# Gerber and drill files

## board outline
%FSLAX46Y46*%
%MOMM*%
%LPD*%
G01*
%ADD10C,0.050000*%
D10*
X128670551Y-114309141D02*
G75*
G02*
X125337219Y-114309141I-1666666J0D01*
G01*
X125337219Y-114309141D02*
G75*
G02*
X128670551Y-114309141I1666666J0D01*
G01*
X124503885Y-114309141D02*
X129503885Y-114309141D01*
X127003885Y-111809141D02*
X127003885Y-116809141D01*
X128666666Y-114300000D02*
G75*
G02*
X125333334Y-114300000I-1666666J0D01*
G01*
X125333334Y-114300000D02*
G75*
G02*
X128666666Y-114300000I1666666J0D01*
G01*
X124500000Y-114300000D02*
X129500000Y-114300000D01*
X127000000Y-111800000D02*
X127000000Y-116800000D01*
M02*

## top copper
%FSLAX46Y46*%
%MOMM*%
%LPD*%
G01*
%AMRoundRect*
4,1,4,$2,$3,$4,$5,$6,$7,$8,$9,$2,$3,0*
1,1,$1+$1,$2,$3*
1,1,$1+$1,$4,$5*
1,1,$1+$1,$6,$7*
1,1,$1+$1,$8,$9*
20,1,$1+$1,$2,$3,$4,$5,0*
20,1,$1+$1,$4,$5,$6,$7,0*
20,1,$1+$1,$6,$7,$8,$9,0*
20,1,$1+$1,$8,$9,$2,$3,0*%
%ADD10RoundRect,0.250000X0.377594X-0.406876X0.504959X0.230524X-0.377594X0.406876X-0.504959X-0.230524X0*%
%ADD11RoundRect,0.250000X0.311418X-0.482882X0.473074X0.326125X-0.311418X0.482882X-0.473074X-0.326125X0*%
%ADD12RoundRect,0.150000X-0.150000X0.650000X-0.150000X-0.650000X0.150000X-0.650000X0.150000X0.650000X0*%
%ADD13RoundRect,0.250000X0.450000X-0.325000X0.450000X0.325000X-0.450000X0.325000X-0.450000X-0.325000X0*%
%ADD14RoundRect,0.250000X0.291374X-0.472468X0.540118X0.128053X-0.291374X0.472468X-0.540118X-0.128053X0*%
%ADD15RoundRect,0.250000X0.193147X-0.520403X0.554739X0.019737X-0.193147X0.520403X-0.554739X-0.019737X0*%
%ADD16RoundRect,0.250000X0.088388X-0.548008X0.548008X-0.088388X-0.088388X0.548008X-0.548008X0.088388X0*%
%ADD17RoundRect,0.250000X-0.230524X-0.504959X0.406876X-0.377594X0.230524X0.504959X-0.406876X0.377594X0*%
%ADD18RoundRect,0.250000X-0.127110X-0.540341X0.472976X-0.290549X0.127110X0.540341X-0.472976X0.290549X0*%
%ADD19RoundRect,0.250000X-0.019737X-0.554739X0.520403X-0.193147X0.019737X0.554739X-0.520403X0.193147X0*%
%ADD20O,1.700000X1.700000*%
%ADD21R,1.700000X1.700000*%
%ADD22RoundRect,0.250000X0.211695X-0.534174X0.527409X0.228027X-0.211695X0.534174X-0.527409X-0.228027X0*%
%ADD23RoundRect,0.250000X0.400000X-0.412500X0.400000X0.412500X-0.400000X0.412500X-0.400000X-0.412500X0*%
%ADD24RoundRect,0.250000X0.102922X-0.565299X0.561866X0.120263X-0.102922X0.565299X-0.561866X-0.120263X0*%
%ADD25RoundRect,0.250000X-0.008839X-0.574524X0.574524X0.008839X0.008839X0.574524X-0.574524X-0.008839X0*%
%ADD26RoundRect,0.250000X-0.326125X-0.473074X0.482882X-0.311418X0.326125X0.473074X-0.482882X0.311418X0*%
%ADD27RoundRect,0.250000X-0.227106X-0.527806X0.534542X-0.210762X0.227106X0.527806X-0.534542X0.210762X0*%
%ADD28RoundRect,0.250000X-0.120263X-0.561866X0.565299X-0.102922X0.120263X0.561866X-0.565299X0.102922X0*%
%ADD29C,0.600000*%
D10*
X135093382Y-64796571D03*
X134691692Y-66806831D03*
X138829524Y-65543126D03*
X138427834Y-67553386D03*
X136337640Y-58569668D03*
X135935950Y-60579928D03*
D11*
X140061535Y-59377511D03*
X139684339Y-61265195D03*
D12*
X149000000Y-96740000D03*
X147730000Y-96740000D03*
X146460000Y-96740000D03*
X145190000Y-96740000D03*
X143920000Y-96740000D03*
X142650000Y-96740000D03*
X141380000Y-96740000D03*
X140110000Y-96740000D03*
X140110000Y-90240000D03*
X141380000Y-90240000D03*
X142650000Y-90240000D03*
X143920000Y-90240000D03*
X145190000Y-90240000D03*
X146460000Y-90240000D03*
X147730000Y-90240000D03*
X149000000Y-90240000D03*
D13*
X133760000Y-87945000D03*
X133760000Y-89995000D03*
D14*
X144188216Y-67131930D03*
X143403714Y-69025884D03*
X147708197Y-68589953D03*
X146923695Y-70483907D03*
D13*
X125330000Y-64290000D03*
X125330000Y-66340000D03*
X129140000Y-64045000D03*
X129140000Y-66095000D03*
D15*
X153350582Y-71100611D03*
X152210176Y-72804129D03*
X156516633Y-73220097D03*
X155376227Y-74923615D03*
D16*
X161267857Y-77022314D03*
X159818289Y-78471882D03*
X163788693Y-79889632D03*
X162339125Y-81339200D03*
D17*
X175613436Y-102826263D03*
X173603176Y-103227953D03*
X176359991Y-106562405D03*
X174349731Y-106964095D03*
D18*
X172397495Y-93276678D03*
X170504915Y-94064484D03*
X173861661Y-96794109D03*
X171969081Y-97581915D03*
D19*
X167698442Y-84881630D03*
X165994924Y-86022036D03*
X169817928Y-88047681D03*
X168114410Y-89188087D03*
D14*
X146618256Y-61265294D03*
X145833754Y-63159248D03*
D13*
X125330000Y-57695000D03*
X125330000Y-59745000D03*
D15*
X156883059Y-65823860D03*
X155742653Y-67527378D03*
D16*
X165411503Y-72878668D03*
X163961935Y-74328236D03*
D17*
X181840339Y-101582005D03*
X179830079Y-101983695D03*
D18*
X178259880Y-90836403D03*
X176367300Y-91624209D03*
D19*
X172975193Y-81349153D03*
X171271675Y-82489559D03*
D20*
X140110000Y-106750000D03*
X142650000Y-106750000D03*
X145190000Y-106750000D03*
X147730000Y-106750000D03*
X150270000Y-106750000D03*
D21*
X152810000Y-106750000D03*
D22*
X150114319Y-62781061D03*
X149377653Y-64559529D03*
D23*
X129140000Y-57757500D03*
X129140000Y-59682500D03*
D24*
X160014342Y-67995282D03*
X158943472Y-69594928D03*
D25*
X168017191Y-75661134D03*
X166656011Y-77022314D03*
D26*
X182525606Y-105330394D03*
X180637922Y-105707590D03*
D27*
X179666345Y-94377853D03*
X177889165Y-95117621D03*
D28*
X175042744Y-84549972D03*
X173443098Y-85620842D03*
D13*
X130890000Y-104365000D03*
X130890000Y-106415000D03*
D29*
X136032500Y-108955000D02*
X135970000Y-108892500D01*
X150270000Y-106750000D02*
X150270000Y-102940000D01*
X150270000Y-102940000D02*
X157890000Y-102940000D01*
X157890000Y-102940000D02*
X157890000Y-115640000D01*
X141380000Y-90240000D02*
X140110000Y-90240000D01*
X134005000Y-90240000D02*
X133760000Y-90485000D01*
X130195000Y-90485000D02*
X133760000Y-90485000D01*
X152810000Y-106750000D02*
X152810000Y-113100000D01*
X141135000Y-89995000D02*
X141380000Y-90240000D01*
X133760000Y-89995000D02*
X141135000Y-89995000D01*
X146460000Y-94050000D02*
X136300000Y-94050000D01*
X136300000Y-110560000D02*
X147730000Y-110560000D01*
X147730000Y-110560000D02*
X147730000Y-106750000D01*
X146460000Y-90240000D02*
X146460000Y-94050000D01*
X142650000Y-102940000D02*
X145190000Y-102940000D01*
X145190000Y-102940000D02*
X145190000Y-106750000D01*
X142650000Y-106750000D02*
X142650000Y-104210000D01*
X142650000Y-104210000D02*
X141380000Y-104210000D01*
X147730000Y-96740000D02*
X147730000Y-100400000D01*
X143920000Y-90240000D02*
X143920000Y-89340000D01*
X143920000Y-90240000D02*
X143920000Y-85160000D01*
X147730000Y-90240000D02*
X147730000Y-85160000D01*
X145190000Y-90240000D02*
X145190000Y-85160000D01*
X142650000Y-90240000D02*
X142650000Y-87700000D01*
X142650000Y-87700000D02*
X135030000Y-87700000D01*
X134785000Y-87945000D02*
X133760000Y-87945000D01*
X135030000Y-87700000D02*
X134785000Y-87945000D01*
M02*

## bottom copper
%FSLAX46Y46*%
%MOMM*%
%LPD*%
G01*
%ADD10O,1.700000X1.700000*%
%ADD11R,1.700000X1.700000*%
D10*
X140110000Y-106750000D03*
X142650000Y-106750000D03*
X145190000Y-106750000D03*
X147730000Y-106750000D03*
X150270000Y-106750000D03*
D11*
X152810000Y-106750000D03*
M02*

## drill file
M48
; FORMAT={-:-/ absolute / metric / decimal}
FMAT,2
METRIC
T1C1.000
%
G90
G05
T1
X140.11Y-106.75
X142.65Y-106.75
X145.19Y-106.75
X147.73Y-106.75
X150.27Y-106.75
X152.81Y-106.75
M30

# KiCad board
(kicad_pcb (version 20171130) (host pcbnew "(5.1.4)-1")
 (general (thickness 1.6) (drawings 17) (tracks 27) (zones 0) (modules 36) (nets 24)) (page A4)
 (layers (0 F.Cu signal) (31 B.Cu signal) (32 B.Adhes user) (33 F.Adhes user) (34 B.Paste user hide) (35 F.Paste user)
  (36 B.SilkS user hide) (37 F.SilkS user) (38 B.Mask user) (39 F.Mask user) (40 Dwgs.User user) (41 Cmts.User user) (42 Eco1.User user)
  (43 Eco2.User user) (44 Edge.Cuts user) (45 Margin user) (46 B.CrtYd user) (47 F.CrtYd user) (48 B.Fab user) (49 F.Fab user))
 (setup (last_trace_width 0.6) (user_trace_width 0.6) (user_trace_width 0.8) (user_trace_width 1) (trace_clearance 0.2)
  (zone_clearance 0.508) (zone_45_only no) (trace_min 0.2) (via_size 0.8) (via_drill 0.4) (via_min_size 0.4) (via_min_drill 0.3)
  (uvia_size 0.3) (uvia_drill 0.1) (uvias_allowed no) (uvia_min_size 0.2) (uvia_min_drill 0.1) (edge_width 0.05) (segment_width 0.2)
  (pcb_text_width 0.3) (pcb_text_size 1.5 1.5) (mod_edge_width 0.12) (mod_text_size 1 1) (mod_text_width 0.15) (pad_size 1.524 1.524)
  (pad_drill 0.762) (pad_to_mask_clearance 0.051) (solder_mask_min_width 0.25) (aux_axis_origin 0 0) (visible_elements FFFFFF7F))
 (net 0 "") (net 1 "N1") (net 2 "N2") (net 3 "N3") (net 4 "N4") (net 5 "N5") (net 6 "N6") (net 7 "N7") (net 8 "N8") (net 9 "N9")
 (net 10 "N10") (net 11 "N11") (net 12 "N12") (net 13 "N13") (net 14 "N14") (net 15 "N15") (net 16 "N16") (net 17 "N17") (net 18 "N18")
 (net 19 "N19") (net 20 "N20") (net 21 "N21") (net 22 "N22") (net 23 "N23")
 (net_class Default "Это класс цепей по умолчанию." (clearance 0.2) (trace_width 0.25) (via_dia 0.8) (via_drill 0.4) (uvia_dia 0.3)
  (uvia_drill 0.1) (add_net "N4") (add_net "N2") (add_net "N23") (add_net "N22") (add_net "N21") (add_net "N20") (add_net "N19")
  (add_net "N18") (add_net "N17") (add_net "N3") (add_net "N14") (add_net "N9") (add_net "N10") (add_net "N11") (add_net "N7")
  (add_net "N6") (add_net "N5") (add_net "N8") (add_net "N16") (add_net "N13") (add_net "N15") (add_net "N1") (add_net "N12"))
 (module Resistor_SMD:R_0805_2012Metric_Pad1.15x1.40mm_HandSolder (layer F.Cu) (at 134.892537 65.801701 78.7)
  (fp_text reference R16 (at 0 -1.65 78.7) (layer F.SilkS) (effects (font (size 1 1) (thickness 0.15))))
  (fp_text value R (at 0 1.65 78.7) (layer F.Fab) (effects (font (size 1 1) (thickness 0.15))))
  (pad 2 smd roundrect (at 1.025 0 78.7) (size 1.15 1.4) (layers F.Cu F.Paste F.Mask) (roundrect_rratio 0.217391) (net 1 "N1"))
  (pad 1 smd roundrect (at -1.025 0 78.7) (size 1.15 1.4) (layers F.Cu F.Paste F.Mask) (roundrect_rratio 0.217391) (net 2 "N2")))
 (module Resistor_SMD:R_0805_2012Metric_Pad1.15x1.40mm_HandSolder (layer F.Cu) (at 138.628679 66.548256 78.7)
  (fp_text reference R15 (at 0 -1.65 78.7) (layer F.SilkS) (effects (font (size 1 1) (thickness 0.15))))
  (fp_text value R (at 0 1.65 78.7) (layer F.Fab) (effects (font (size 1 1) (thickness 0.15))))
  (pad 2 smd roundrect (at 1.025 0 78.7) (size 1.15 1.4) (layers F.Cu F.Paste F.Mask) (roundrect_rratio 0.217391) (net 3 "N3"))
  (pad 1 smd roundrect (at -1.025 0 78.7) (size 1.15 1.4) (layers F.Cu F.Paste F.Mask) (roundrect_rratio 0.217391) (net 2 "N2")))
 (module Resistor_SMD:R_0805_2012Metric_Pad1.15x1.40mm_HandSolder (layer F.Cu) (at 136.136795 59.574798 78.7)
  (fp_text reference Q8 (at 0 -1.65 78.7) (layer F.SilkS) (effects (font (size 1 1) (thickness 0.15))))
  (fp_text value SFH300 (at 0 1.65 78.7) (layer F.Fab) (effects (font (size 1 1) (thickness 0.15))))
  (pad 2 smd roundrect (at 1.025 0 78.7) (size 1.15 1.4) (layers F.Cu F.Paste F.Mask) (roundrect_rratio 0.217391) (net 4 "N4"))
  (pad 1 smd roundrect (at -1.025 0 78.7) (size 1.15 1.4) (layers F.Cu F.Paste F.Mask) (roundrect_rratio 0.217391) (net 1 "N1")))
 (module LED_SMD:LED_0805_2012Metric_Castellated (layer F.Cu) (at 139.872937 60.321353 78.7)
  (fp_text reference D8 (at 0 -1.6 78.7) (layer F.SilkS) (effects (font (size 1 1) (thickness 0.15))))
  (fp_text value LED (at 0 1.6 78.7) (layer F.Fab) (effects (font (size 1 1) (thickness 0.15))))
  (pad 2 smd roundrect (at 0.9625 0 78.7) (size 1.325 1.3) (layers F.Cu F.Paste F.Mask) (roundrect_rratio 0.192308) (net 4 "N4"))
  (pad 1 smd roundrect (at -0.9625 0 78.7) (size 1.325 1.3) (layers F.Cu F.Paste F.Mask) (roundrect_rratio 0.192308) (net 3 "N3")))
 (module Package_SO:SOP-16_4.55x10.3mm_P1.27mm (layer F.Cu) (at 144.555 93.49 270)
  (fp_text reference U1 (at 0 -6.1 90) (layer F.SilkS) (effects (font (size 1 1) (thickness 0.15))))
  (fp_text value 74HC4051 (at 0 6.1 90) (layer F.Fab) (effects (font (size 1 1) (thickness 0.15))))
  (pad 16 smd roundrect (at 3.25 -4.445 270) (size 1.6 0.6) (layers F.Cu F.Paste F.Mask) (roundrect_rratio 0.25) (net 4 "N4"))
  (pad 15 smd roundrect (at 3.25 -3.175 270) (size 1.6 0.6) (layers F.Cu F.Paste F.Mask) (roundrect_rratio 0.25) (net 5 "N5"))
  (pad 14 smd roundrect (at 3.25 -1.905 270) (size 1.6 0.6) (layers F.Cu F.Paste F.Mask) (roundrect_rratio 0.25) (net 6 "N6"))
  (pad 13 smd roundrect (at 3.25 -0.635 270) (size 1.6 0.6) (layers F.Cu F.Paste F.Mask) (roundrect_rratio 0.25) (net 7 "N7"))
  (pad 12 smd roundrect (at 3.25 0.635 270) (size 1.6 0.6) (layers F.Cu F.Paste F.Mask) (roundrect_rratio 0.25) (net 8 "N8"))
  (pad 11 smd roundrect (at 3.25 1.905 270) (size 1.6 0.6) (layers F.Cu F.Paste F.Mask) (roundrect_rratio 0.25) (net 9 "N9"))
  (pad 10 smd roundrect (at 3.25 3.175 270) (size 1.6 0.6) (layers F.Cu F.Paste F.Mask) (roundrect_rratio 0.25) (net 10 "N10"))
  (pad 9 smd roundrect (at 3.25 4.445 270) (size 1.6 0.6) (layers F.Cu F.Paste F.Mask) (roundrect_rratio 0.25) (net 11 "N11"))
  (pad 8 smd roundrect (at -3.25 4.445 270) (size 1.6 0.6) (layers F.Cu F.Paste F.Mask) (roundrect_rratio 0.25) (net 2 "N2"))
  (pad 7 smd roundrect (at -3.25 3.175 270) (size 1.6 0.6) (layers F.Cu F.Paste F.Mask) (roundrect_rratio 0.25) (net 2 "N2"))
  (pad 6 smd roundrect (at -3.25 1.905 270) (size 1.6 0.6) (layers F.Cu F.Paste F.Mask) (roundrect_rratio 0.25) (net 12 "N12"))
  (pad 5 smd roundrect (at -3.25 0.635 270) (size 1.6 0.6) (layers F.Cu F.Paste F.Mask) (roundrect_rratio 0.25) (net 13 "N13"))
  (pad 4 smd roundrect (at -3.25 -0.635 270) (size 1.6 0.6) (layers F.Cu F.Paste F.Mask) (roundrect_rratio 0.25) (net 1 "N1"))
  (pad 3 smd roundrect (at -3.25 -1.905 270) (size 1.6 0.6) (layers F.Cu F.Paste F.Mask) (roundrect_rratio 0.25) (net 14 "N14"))
  (pad 2 smd roundrect (at -3.25 -3.175 270) (size 1.6 0.6) (layers F.Cu F.Paste F.Mask) (roundrect_rratio 0.25) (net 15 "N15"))
  (pad 1 smd roundrect (at -3.25 -4.445 270) (size 1.6 0.6) (layers F.Cu F.Paste F.Mask) (roundrect_rratio 0.25) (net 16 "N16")))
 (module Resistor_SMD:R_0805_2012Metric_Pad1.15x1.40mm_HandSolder (layer F.Cu) (at 133.76 88.97 90)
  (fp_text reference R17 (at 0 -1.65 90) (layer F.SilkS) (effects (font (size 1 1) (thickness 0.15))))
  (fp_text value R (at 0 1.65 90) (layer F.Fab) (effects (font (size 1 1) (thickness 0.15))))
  (pad 2 smd roundrect (at 1.025 0 90) (size 1.15 1.4) (layers F.Cu F.Paste F.Mask) (roundrect_rratio 0.217391) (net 12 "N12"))
  (pad 1 smd roundrect (at -1.025 0 90) (size 1.15 1.4) (layers F.Cu F.Paste F.Mask) (roundrect_rratio 0.217391) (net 2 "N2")))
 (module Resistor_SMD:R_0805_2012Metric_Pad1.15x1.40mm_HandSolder (layer F.Cu) (at 143.795965 68.078907 67.5)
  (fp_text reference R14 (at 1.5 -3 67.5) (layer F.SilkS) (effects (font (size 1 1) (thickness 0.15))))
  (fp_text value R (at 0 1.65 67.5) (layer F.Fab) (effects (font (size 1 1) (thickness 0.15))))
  (pad 2 smd roundrect (at 1.025 0 67.5) (size 1.15 1.4) (layers F.Cu F.Paste F.Mask) (roundrect_rratio 0.217391) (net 15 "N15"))
  (pad 1 smd roundrect (at -1.025 0 67.5) (size 1.15 1.4) (layers F.Cu F.Paste F.Mask) (roundrect_rratio 0.217391) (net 2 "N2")))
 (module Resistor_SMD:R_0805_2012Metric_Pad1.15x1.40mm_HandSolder (layer F.Cu) (at 147.315946 69.53693 67.5)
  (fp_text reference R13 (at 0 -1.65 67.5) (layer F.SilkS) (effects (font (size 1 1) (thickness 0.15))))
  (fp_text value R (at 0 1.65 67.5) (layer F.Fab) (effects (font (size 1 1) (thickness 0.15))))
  (pad 2 smd roundrect (at 1.025 0 67.5) (size 1.15 1.4) (layers F.Cu F.Paste F.Mask) (roundrect_rratio 0.217391) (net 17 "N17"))
  (pad 1 smd roundrect (at -1.025 0 67.5) (size 1.15 1.4) (layers F.Cu F.Paste F.Mask) (roundrect_rratio 0.217391) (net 2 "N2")))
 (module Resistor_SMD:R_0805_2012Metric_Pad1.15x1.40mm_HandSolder (layer F.Cu) (at 125.33 65.315 90)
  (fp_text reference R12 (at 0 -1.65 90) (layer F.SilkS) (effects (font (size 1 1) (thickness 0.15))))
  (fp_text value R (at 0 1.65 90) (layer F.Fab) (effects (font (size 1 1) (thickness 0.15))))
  (pad 2 smd roundrect (at 1.025 0 90) (size 1.15 1.4) (layers F.Cu F.Paste F.Mask) (roundrect_rratio 0.217391) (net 13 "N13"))
  (pad 1 smd roundrect (at -1.025 0 90) (size 1.15 1.4) (layers F.Cu F.Paste F.Mask) (roundrect_rratio 0.217391) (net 2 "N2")))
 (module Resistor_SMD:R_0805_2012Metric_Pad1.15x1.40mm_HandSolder (layer F.Cu) (at 129.14 65.07 90)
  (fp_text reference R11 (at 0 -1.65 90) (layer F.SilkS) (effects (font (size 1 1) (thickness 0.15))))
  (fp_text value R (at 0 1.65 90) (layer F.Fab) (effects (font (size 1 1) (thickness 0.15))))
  (pad 2 smd roundrect (at 1.025 0 90) (size 1.15 1.4) (layers F.Cu F.Paste F.Mask) (roundrect_rratio 0.217391) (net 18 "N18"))
  (pad 1 smd roundrect (at -1.025 0 90) (size 1.15 1.4) (layers F.Cu F.Paste F.Mask) (roundrect_rratio 0.217391) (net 2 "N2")))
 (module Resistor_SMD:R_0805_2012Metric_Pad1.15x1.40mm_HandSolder (layer F.Cu) (at 152.780379 71.95237 56.2)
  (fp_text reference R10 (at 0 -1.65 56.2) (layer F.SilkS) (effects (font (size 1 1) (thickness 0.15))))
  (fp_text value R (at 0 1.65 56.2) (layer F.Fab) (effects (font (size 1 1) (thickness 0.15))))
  (pad 2 smd roundrect (at 1.025 0 56.2) (size 1.15 1.4) (layers F.Cu F.Paste F.Mask) (roundrect_rratio 0.217391) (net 16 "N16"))
  (pad 1 smd roundrect (at -1.025 0 56.2) (size 1.15 1.4) (layers F.Cu F.Paste F.Mask) (roundrect_rratio 0.217391) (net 2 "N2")))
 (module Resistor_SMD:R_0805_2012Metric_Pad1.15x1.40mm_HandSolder (layer F.Cu) (at 155.94643 74.071856 56.2)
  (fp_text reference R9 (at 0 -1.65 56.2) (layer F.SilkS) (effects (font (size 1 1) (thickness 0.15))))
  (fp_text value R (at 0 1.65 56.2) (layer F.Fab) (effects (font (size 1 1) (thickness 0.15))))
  (pad 2 smd roundrect (at 1.025 0 56.2) (size 1.15 1.4) (layers F.Cu F.Paste F.Mask) (roundrect_rratio 0.217391) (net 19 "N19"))
  (pad 1 smd roundrect (at -1.025 0 56.2) (size 1.15 1.4) (layers F.Cu F.Paste F.Mask) (roundrect_rratio 0.217391) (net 2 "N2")))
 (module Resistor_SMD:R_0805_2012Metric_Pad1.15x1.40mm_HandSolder (layer F.Cu) (at 160.543073 77.747098 45)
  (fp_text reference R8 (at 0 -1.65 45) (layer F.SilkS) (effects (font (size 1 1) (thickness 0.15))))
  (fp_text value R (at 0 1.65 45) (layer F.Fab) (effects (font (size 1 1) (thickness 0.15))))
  (pad 2 smd roundrect (at 1.025 0 45) (size 1.15 1.4) (layers F.Cu F.Paste F.Mask) (roundrect_rratio 0.217391) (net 8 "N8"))
  (pad 1 smd roundrect (at -1.025 0 45) (size 1.15 1.4) (layers F.Cu F.Paste F.Mask) (roundrect_rratio 0.217391) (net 2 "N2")))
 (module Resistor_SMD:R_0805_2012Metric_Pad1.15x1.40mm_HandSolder (layer F.Cu) (at 163.063909 80.614416 45)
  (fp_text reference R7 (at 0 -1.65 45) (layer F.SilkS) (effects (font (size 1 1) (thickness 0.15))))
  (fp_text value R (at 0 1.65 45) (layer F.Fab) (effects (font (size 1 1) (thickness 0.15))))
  (pad 2 smd roundrect (at 1.025 0 45) (size 1.15 1.4) (layers F.Cu F.Paste F.Mask) (roundrect_rratio 0.217391) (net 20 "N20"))
  (pad 1 smd roundrect (at -1.025 0 45) (size 1.15 1.4) (layers F.Cu F.Paste F.Mask) (roundrect_rratio 0.217391) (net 2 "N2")))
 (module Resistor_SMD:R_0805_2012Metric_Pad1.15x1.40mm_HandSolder (layer F.Cu) (at 174.608306 103.027108 11.3)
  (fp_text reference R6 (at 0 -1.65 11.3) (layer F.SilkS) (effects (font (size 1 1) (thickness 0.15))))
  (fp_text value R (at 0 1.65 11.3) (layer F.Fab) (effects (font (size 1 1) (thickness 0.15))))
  (pad 2 smd roundrect (at 1.025 0 11.3) (size 1.15 1.4) (layers F.Cu F.Paste F.Mask) (roundrect_rratio 0.217391) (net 5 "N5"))
  (pad 1 smd roundrect (at -1.025 0 11.3) (size 1.15 1.4) (layers F.Cu F.Paste F.Mask) (roundrect_rratio 0.217391) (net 2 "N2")))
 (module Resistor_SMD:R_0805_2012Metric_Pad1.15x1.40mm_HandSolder (layer F.Cu) (at 175.354861 106.76325 11.3)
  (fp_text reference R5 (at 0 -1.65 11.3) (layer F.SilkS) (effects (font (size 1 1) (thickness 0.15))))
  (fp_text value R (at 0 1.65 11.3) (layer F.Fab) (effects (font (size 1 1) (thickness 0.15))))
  (pad 2 smd roundrect (at 1.025 0 11.3) (size 1.15 1.4) (layers F.Cu F.Paste F.Mask) (roundrect_rratio 0.217391) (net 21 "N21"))
  (pad 1 smd roundrect (at -1.025 0 11.3) (size 1.15 1.4) (layers F.Cu F.Paste F.Mask) (roundrect_rratio 0.217391) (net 2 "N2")))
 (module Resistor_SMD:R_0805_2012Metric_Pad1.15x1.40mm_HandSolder (layer F.Cu) (at 171.451205 93.670581 22.6)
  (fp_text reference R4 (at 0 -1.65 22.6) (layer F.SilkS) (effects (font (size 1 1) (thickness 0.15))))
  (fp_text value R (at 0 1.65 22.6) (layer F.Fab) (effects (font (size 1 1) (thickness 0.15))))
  (pad 2 smd roundrect (at 1.025 0 22.6) (size 1.15 1.4) (layers F.Cu F.Paste F.Mask) (roundrect_rratio 0.217391) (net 6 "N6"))
  (pad 1 smd roundrect (at -1.025 0 22.6) (size 1.15 1.4) (layers F.Cu F.Paste F.Mask) (roundrect_rratio 0.217391) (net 2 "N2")))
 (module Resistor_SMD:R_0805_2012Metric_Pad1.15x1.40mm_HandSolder (layer F.Cu) (at 172.915371 97.188012 22.6)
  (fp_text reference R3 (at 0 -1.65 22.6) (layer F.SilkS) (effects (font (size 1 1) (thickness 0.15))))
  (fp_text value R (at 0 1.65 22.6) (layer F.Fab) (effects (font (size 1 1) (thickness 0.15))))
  (pad 2 smd roundrect (at 1.025 0 22.6) (size 1.15 1.4) (layers F.Cu F.Paste F.Mask) (roundrect_rratio 0.217391) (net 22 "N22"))
  (pad 1 smd roundrect (at -1.025 0 22.6) (size 1.15 1.4) (layers F.Cu F.Paste F.Mask) (roundrect_rratio 0.217391) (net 2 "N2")))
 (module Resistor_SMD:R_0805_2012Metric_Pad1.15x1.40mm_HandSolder (layer F.Cu) (at 166.846683 85.451833 33.8)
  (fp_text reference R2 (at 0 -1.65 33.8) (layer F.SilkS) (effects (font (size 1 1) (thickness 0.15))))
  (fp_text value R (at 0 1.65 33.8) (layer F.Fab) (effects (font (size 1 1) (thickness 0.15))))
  (pad 2 smd roundrect (at 1.025 0 33.8) (size 1.15 1.4) (layers F.Cu F.Paste F.Mask) (roundrect_rratio 0.217391) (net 7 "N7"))
  (pad 1 smd roundrect (at -1.025 0 33.8) (size 1.15 1.4) (layers F.Cu F.Paste F.Mask) (roundrect_rratio 0.217391) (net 2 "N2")))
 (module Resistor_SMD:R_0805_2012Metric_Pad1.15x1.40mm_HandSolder (layer F.Cu) (at 168.966169 88.617884 33.8)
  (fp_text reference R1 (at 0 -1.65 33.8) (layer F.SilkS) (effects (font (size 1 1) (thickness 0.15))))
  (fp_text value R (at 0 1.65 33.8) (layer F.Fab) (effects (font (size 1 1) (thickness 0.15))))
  (pad 2 smd roundrect (at 1.025 0 33.8) (size 1.15 1.4) (layers F.Cu F.Paste F.Mask) (roundrect_rratio 0.217391) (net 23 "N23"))
  (pad 1 smd roundrect (at -1.025 0 33.8) (size 1.15 1.4) (layers F.Cu F.Paste F.Mask) (roundrect_rratio 0.217391) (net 2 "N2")))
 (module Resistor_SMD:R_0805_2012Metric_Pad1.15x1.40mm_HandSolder (layer F.Cu) (at 146.226005 62.212271 67.5)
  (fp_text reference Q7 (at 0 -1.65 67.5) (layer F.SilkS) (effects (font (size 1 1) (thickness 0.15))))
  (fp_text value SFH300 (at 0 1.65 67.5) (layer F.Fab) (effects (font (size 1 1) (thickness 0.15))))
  (pad 2 smd roundrect (at 1.025 0 67.5) (size 1.15 1.4) (layers F.Cu F.Paste F.Mask) (roundrect_rratio 0.217391) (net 4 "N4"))
  (pad 1 smd roundrect (at -1.025 0 67.5) (size 1.15 1.4) (layers F.Cu F.Paste F.Mask) (roundrect_rratio 0.217391) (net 15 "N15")))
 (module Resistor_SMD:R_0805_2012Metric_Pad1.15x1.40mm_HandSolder (layer F.Cu) (at 125.33 58.72 90)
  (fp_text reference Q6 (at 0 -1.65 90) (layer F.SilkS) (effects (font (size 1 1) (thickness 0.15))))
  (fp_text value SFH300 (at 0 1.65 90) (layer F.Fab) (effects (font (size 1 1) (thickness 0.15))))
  (pad 2 smd roundrect (at 1.025 0 90) (size 1.15 1.4) (layers F.Cu F.Paste F.Mask) (roundrect_rratio 0.217391) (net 4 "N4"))
  (pad 1 smd roundrect (at -1.025 0 90) (size 1.15 1.4) (layers F.Cu F.Paste F.Mask) (roundrect_rratio 0.217391) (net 13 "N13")))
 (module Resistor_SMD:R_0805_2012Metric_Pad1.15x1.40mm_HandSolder (layer F.Cu) (at 156.312856 66.675619 56.2)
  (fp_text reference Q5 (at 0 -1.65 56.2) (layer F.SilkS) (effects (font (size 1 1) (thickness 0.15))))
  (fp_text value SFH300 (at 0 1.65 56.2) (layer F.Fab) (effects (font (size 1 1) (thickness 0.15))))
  (pad 2 smd roundrect (at 1.025 0 56.2) (size 1.15 1.4) (layers F.Cu F.Paste F.Mask) (roundrect_rratio 0.217391) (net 4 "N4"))
  (pad 1 smd roundrect (at -1.025 0 56.2) (size 1.15 1.4) (layers F.Cu F.Paste F.Mask) (roundrect_rratio 0.217391) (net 16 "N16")))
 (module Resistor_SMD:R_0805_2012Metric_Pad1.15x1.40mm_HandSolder (layer F.Cu) (at 164.686719 73.603452 45)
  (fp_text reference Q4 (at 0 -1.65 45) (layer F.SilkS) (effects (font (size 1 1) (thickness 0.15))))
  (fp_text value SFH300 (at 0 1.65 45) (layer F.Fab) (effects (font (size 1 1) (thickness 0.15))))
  (pad 2 smd roundrect (at 1.025 0 45) (size 1.15 1.4) (layers F.Cu F.Paste F.Mask) (roundrect_rratio 0.217391) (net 4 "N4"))
  (pad 1 smd roundrect (at -1.025 0 45) (size 1.15 1.4) (layers F.Cu F.Paste F.Mask) (roundrect_rratio 0.217391) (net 8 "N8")))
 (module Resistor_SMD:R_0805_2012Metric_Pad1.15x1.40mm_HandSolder (layer F.Cu) (at 180.835209 101.78285 11.3)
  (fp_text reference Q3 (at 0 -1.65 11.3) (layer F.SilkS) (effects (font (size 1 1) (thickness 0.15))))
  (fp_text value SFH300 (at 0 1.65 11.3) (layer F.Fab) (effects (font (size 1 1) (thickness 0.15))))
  (pad 2 smd roundrect (at 1.025 0 11.3) (size 1.15 1.4) (layers F.Cu F.Paste F.Mask) (roundrect_rratio 0.217391) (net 4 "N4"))
  (pad 1 smd roundrect (at -1.025 0 11.3) (size 1.15 1.4) (layers F.Cu F.Paste F.Mask) (roundrect_rratio 0.217391) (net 5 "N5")))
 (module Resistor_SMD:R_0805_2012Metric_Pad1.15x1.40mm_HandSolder (layer F.Cu) (at 177.31359 91.230306 22.6)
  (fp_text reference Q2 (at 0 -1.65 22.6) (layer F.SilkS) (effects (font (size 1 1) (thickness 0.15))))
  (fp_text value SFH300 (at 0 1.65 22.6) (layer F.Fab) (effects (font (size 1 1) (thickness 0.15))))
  (pad 2 smd roundrect (at 1.025 0 22.6) (size 1.15 1.4) (layers F.Cu F.Paste F.Mask) (roundrect_rratio 0.217391) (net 4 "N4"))
  (pad 1 smd roundrect (at -1.025 0 22.6) (size 1.15 1.4) (layers F.Cu F.Paste F.Mask) (roundrect_rratio 0.217391) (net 6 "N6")))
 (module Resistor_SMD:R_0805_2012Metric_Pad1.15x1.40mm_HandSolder (layer F.Cu) (at 172.123434 81.919356 33.8)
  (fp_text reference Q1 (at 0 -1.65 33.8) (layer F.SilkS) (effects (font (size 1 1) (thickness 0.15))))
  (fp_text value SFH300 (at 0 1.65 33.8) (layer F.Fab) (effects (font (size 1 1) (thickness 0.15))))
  (pad 2 smd roundrect (at 1.025 0 33.8) (size 1.15 1.4) (layers F.Cu F.Paste F.Mask) (roundrect_rratio 0.217391) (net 4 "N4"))
  (pad 1 smd roundrect (at -1.025 0 33.8) (size 1.15 1.4) (layers F.Cu F.Paste F.Mask) (roundrect_rratio 0.217391) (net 7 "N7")))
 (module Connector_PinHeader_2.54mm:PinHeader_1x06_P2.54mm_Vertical (layer F.Cu) (at 152.81 106.75 270)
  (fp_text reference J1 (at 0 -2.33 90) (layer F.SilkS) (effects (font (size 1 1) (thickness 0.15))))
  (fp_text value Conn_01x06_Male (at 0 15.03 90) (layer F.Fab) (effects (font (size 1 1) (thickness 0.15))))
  (pad 6 thru_hole oval (at 0 12.7 270) (size 1.7 1.7) (drill 1) (layers *.Cu *.Mask) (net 11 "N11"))
  (pad 5 thru_hole oval (at 0 10.16 270) (size 1.7 1.7) (drill 1) (layers *.Cu *.Mask) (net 10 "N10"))
  (pad 4 thru_hole oval (at 0 7.62 270) (size 1.7 1.7) (drill 1) (layers *.Cu *.Mask) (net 9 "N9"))
  (pad 3 thru_hole oval (at 0 5.08 270) (size 1.7 1.7) (drill 1) (layers *.Cu *.Mask) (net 14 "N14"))
  (pad 2 thru_hole oval (at 0 2.54 270) (size 1.7 1.7) (drill 1) (layers *.Cu *.Mask) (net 4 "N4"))
  (pad 1 thru_hole rect (at 0 0 270) (size 1.7 1.7) (drill 1) (layers *.Cu *.Mask) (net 2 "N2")))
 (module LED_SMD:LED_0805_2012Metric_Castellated (layer F.Cu) (at 149.745986 63.670295 67.5)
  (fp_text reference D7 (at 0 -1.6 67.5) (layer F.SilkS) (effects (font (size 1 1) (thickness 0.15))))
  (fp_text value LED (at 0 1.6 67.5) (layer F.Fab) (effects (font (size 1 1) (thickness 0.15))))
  (pad 2 smd roundrect (at 0.9625 0 67.5) (size 1.325 1.3) (layers F.Cu F.Paste F.Mask) (roundrect_rratio 0.192308) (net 4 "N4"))
  (pad 1 smd roundrect (at -0.9625 0 67.5) (size 1.325 1.3) (layers F.Cu F.Paste F.Mask) (roundrect_rratio 0.192308) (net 17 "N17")))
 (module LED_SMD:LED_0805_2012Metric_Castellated (layer F.Cu) (at 129.14 58.72 90)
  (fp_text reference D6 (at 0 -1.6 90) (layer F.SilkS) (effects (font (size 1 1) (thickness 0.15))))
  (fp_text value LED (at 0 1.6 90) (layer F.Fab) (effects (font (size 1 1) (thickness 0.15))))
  (pad 2 smd roundrect (at 0.9625 0 90) (size 1.325 1.3) (layers F.Cu F.Paste F.Mask) (roundrect_rratio 0.192308) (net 4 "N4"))
  (pad 1 smd roundrect (at -0.9625 0 90) (size 1.325 1.3) (layers F.Cu F.Paste F.Mask) (roundrect_rratio 0.192308) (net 18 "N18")))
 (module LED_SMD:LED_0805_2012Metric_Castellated (layer F.Cu) (at 159.478907 68.795105 56.2)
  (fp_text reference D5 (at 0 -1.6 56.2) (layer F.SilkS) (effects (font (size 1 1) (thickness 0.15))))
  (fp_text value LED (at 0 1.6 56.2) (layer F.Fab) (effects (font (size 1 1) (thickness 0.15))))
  (pad 2 smd roundrect (at 0.9625 0 56.2) (size 1.325 1.3) (layers F.Cu F.Paste F.Mask) (roundrect_rratio 0.192308) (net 4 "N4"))
  (pad 1 smd roundrect (at -0.9625 0 56.2) (size 1.325 1.3) (layers F.Cu F.Paste F.Mask) (roundrect_rratio 0.192308) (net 19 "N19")))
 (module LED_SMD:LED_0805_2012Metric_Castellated (layer F.Cu) (at 167.336601 76.341724 45)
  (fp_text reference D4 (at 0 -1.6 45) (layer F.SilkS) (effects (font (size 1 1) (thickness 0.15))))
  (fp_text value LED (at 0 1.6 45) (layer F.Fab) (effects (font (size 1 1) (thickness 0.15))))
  (pad 2 smd roundrect (at 0.9625 0 45) (size 1.325 1.3) (layers F.Cu F.Paste F.Mask) (roundrect_rratio 0.192308) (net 4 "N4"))
  (pad 1 smd roundrect (at -0.9625 0 45) (size 1.325 1.3) (layers F.Cu F.Paste F.Mask) (roundrect_rratio 0.192308) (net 20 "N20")))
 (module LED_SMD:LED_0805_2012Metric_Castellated (layer F.Cu) (at 181.581764 105.518992 11.3)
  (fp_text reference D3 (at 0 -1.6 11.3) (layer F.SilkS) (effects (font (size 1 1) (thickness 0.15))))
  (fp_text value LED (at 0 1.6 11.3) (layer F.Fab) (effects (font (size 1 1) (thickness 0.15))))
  (pad 2 smd roundrect (at 0.9625 0 11.3) (size 1.325 1.3) (layers F.Cu F.Paste F.Mask) (roundrect_rratio 0.192308) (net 4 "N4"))
  (pad 1 smd roundrect (at -0.9625 0 11.3) (size 1.325 1.3) (layers F.Cu F.Paste F.Mask) (roundrect_rratio 0.192308) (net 21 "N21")))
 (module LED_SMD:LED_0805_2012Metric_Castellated (layer F.Cu) (at 178.777755 94.747737 22.6)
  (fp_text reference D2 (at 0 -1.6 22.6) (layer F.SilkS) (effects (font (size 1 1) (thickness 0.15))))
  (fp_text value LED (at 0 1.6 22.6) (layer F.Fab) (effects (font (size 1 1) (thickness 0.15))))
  (pad 2 smd roundrect (at 0.9625 0 22.6) (size 1.325 1.3) (layers F.Cu F.Paste F.Mask) (roundrect_rratio 0.192308) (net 4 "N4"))
  (pad 1 smd roundrect (at -0.9625 0 22.6) (size 1.325 1.3) (layers F.Cu F.Paste F.Mask) (roundrect_rratio 0.192308) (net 22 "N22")))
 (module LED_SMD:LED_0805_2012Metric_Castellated (layer F.Cu) (at 174.242921 85.085407 33.8)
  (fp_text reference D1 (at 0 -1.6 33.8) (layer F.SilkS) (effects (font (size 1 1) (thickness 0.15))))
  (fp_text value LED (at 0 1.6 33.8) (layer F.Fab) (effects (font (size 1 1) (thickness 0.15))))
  (pad 2 smd roundrect (at 0.9625 0 33.8) (size 1.325 1.3) (layers F.Cu F.Paste F.Mask) (roundrect_rratio 0.192308) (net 4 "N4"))
  (pad 1 smd roundrect (at -0.9625 0 33.8) (size 1.325 1.3) (layers F.Cu F.Paste F.Mask) (roundrect_rratio 0.192308) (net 23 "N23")))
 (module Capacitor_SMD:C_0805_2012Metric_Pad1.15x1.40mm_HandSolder (layer F.Cu) (at 130.89 105.39 90)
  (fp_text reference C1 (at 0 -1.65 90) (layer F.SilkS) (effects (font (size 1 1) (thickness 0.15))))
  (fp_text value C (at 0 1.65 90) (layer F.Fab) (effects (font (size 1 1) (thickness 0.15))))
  (pad 2 smd roundrect (at 1.025 0 90) (size 1.15 1.4) (layers F.Cu F.Paste F.Mask) (roundrect_rratio 0.217391) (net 2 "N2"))
  (pad 1 smd roundrect (at -1.025 0 90) (size 1.15 1.4) (layers F.Cu F.Paste F.Mask) (roundrect_rratio 0.217391) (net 4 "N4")))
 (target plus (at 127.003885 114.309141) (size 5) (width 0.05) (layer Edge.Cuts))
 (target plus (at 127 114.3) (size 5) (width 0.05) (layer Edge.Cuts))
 (segment (start 136.0325 108.955) (end 135.97 108.8925) (width 0.6) (layer F.Cu) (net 4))
 (segment (start 150.27 106.75) (end 150.27 102.94) (width 0.6) (layer F.Cu) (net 4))
 (segment (start 150.27 102.94) (end 157.89 102.94) (width 0.6) (layer F.Cu) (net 4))
 (segment (start 157.89 102.94) (end 157.89 115.64) (width 0.6) (layer F.Cu) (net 4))
 (segment (start 141.38 90.24) (end 140.11 90.24) (width 0.6) (layer F.Cu) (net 2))
 (segment (start 134.005 90.24) (end 133.76 90.485) (width 0.6) (layer F.Cu) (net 2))
 (segment (start 130.195 90.485) (end 133.76 90.485) (width 0.6) (layer F.Cu) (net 2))
 (segment (start 152.81 106.75) (end 152.81 113.1) (width 0.6) (layer F.Cu) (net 2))
 (segment (start 141.135 89.995) (end 141.38 90.24) (width 0.6) (layer F.Cu) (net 2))
 (segment (start 133.76 89.995) (end 141.135 89.995) (width 0.6) (layer F.Cu) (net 2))
 (segment (start 146.46 94.05) (end 136.3 94.05) (width 0.6) (layer F.Cu) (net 14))
 (segment (start 136.3 110.56) (end 147.73 110.56) (width 0.6) (layer F.Cu) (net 14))
 (segment (start 147.73 110.56) (end 147.73 106.75) (width 0.6) (layer F.Cu) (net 14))
 (segment (start 146.46 90.24) (end 146.46 94.05) (width 0.6) (layer F.Cu) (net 14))
 (segment (start 142.65 102.94) (end 145.19 102.94) (width 0.6) (layer F.Cu) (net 9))
 (segment (start 145.19 102.94) (end 145.19 106.75) (width 0.6) (layer F.Cu) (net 9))
 (segment (start 142.65 106.75) (end 142.65 104.21) (width 0.6) (layer F.Cu) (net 10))
 (segment (start 142.65 104.21) (end 141.38 104.21) (width 0.6) (layer F.Cu) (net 10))
 (segment (start 147.73 96.74) (end 147.73 100.4) (width 0.6) (layer F.Cu) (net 5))
 (segment (start 143.92 90.24) (end 143.92 89.34) (width 0.6) (layer F.Cu) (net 13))
 (segment (start 143.92 90.24) (end 143.92 85.16) (width 0.6) (layer F.Cu) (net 13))
 (segment (start 147.73 90.24) (end 147.73 85.16) (width 0.6) (layer F.Cu) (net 15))
 (segment (start 145.19 90.24) (end 145.19 85.16) (width 0.6) (layer F.Cu) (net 1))
 (segment (start 142.65 90.24) (end 142.65 87.7) (width 0.6) (layer F.Cu) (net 12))
 (segment (start 142.65 87.7) (end 135.03 87.7) (width 0.6) (layer F.Cu) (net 12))
 (segment (start 134.785 87.945) (end 133.76 87.945) (width 0.6) (layer F.Cu) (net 12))
 (segment (start 135.03 87.7) (end 134.785 87.945) (width 0.6) (layer F.Cu) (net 12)))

